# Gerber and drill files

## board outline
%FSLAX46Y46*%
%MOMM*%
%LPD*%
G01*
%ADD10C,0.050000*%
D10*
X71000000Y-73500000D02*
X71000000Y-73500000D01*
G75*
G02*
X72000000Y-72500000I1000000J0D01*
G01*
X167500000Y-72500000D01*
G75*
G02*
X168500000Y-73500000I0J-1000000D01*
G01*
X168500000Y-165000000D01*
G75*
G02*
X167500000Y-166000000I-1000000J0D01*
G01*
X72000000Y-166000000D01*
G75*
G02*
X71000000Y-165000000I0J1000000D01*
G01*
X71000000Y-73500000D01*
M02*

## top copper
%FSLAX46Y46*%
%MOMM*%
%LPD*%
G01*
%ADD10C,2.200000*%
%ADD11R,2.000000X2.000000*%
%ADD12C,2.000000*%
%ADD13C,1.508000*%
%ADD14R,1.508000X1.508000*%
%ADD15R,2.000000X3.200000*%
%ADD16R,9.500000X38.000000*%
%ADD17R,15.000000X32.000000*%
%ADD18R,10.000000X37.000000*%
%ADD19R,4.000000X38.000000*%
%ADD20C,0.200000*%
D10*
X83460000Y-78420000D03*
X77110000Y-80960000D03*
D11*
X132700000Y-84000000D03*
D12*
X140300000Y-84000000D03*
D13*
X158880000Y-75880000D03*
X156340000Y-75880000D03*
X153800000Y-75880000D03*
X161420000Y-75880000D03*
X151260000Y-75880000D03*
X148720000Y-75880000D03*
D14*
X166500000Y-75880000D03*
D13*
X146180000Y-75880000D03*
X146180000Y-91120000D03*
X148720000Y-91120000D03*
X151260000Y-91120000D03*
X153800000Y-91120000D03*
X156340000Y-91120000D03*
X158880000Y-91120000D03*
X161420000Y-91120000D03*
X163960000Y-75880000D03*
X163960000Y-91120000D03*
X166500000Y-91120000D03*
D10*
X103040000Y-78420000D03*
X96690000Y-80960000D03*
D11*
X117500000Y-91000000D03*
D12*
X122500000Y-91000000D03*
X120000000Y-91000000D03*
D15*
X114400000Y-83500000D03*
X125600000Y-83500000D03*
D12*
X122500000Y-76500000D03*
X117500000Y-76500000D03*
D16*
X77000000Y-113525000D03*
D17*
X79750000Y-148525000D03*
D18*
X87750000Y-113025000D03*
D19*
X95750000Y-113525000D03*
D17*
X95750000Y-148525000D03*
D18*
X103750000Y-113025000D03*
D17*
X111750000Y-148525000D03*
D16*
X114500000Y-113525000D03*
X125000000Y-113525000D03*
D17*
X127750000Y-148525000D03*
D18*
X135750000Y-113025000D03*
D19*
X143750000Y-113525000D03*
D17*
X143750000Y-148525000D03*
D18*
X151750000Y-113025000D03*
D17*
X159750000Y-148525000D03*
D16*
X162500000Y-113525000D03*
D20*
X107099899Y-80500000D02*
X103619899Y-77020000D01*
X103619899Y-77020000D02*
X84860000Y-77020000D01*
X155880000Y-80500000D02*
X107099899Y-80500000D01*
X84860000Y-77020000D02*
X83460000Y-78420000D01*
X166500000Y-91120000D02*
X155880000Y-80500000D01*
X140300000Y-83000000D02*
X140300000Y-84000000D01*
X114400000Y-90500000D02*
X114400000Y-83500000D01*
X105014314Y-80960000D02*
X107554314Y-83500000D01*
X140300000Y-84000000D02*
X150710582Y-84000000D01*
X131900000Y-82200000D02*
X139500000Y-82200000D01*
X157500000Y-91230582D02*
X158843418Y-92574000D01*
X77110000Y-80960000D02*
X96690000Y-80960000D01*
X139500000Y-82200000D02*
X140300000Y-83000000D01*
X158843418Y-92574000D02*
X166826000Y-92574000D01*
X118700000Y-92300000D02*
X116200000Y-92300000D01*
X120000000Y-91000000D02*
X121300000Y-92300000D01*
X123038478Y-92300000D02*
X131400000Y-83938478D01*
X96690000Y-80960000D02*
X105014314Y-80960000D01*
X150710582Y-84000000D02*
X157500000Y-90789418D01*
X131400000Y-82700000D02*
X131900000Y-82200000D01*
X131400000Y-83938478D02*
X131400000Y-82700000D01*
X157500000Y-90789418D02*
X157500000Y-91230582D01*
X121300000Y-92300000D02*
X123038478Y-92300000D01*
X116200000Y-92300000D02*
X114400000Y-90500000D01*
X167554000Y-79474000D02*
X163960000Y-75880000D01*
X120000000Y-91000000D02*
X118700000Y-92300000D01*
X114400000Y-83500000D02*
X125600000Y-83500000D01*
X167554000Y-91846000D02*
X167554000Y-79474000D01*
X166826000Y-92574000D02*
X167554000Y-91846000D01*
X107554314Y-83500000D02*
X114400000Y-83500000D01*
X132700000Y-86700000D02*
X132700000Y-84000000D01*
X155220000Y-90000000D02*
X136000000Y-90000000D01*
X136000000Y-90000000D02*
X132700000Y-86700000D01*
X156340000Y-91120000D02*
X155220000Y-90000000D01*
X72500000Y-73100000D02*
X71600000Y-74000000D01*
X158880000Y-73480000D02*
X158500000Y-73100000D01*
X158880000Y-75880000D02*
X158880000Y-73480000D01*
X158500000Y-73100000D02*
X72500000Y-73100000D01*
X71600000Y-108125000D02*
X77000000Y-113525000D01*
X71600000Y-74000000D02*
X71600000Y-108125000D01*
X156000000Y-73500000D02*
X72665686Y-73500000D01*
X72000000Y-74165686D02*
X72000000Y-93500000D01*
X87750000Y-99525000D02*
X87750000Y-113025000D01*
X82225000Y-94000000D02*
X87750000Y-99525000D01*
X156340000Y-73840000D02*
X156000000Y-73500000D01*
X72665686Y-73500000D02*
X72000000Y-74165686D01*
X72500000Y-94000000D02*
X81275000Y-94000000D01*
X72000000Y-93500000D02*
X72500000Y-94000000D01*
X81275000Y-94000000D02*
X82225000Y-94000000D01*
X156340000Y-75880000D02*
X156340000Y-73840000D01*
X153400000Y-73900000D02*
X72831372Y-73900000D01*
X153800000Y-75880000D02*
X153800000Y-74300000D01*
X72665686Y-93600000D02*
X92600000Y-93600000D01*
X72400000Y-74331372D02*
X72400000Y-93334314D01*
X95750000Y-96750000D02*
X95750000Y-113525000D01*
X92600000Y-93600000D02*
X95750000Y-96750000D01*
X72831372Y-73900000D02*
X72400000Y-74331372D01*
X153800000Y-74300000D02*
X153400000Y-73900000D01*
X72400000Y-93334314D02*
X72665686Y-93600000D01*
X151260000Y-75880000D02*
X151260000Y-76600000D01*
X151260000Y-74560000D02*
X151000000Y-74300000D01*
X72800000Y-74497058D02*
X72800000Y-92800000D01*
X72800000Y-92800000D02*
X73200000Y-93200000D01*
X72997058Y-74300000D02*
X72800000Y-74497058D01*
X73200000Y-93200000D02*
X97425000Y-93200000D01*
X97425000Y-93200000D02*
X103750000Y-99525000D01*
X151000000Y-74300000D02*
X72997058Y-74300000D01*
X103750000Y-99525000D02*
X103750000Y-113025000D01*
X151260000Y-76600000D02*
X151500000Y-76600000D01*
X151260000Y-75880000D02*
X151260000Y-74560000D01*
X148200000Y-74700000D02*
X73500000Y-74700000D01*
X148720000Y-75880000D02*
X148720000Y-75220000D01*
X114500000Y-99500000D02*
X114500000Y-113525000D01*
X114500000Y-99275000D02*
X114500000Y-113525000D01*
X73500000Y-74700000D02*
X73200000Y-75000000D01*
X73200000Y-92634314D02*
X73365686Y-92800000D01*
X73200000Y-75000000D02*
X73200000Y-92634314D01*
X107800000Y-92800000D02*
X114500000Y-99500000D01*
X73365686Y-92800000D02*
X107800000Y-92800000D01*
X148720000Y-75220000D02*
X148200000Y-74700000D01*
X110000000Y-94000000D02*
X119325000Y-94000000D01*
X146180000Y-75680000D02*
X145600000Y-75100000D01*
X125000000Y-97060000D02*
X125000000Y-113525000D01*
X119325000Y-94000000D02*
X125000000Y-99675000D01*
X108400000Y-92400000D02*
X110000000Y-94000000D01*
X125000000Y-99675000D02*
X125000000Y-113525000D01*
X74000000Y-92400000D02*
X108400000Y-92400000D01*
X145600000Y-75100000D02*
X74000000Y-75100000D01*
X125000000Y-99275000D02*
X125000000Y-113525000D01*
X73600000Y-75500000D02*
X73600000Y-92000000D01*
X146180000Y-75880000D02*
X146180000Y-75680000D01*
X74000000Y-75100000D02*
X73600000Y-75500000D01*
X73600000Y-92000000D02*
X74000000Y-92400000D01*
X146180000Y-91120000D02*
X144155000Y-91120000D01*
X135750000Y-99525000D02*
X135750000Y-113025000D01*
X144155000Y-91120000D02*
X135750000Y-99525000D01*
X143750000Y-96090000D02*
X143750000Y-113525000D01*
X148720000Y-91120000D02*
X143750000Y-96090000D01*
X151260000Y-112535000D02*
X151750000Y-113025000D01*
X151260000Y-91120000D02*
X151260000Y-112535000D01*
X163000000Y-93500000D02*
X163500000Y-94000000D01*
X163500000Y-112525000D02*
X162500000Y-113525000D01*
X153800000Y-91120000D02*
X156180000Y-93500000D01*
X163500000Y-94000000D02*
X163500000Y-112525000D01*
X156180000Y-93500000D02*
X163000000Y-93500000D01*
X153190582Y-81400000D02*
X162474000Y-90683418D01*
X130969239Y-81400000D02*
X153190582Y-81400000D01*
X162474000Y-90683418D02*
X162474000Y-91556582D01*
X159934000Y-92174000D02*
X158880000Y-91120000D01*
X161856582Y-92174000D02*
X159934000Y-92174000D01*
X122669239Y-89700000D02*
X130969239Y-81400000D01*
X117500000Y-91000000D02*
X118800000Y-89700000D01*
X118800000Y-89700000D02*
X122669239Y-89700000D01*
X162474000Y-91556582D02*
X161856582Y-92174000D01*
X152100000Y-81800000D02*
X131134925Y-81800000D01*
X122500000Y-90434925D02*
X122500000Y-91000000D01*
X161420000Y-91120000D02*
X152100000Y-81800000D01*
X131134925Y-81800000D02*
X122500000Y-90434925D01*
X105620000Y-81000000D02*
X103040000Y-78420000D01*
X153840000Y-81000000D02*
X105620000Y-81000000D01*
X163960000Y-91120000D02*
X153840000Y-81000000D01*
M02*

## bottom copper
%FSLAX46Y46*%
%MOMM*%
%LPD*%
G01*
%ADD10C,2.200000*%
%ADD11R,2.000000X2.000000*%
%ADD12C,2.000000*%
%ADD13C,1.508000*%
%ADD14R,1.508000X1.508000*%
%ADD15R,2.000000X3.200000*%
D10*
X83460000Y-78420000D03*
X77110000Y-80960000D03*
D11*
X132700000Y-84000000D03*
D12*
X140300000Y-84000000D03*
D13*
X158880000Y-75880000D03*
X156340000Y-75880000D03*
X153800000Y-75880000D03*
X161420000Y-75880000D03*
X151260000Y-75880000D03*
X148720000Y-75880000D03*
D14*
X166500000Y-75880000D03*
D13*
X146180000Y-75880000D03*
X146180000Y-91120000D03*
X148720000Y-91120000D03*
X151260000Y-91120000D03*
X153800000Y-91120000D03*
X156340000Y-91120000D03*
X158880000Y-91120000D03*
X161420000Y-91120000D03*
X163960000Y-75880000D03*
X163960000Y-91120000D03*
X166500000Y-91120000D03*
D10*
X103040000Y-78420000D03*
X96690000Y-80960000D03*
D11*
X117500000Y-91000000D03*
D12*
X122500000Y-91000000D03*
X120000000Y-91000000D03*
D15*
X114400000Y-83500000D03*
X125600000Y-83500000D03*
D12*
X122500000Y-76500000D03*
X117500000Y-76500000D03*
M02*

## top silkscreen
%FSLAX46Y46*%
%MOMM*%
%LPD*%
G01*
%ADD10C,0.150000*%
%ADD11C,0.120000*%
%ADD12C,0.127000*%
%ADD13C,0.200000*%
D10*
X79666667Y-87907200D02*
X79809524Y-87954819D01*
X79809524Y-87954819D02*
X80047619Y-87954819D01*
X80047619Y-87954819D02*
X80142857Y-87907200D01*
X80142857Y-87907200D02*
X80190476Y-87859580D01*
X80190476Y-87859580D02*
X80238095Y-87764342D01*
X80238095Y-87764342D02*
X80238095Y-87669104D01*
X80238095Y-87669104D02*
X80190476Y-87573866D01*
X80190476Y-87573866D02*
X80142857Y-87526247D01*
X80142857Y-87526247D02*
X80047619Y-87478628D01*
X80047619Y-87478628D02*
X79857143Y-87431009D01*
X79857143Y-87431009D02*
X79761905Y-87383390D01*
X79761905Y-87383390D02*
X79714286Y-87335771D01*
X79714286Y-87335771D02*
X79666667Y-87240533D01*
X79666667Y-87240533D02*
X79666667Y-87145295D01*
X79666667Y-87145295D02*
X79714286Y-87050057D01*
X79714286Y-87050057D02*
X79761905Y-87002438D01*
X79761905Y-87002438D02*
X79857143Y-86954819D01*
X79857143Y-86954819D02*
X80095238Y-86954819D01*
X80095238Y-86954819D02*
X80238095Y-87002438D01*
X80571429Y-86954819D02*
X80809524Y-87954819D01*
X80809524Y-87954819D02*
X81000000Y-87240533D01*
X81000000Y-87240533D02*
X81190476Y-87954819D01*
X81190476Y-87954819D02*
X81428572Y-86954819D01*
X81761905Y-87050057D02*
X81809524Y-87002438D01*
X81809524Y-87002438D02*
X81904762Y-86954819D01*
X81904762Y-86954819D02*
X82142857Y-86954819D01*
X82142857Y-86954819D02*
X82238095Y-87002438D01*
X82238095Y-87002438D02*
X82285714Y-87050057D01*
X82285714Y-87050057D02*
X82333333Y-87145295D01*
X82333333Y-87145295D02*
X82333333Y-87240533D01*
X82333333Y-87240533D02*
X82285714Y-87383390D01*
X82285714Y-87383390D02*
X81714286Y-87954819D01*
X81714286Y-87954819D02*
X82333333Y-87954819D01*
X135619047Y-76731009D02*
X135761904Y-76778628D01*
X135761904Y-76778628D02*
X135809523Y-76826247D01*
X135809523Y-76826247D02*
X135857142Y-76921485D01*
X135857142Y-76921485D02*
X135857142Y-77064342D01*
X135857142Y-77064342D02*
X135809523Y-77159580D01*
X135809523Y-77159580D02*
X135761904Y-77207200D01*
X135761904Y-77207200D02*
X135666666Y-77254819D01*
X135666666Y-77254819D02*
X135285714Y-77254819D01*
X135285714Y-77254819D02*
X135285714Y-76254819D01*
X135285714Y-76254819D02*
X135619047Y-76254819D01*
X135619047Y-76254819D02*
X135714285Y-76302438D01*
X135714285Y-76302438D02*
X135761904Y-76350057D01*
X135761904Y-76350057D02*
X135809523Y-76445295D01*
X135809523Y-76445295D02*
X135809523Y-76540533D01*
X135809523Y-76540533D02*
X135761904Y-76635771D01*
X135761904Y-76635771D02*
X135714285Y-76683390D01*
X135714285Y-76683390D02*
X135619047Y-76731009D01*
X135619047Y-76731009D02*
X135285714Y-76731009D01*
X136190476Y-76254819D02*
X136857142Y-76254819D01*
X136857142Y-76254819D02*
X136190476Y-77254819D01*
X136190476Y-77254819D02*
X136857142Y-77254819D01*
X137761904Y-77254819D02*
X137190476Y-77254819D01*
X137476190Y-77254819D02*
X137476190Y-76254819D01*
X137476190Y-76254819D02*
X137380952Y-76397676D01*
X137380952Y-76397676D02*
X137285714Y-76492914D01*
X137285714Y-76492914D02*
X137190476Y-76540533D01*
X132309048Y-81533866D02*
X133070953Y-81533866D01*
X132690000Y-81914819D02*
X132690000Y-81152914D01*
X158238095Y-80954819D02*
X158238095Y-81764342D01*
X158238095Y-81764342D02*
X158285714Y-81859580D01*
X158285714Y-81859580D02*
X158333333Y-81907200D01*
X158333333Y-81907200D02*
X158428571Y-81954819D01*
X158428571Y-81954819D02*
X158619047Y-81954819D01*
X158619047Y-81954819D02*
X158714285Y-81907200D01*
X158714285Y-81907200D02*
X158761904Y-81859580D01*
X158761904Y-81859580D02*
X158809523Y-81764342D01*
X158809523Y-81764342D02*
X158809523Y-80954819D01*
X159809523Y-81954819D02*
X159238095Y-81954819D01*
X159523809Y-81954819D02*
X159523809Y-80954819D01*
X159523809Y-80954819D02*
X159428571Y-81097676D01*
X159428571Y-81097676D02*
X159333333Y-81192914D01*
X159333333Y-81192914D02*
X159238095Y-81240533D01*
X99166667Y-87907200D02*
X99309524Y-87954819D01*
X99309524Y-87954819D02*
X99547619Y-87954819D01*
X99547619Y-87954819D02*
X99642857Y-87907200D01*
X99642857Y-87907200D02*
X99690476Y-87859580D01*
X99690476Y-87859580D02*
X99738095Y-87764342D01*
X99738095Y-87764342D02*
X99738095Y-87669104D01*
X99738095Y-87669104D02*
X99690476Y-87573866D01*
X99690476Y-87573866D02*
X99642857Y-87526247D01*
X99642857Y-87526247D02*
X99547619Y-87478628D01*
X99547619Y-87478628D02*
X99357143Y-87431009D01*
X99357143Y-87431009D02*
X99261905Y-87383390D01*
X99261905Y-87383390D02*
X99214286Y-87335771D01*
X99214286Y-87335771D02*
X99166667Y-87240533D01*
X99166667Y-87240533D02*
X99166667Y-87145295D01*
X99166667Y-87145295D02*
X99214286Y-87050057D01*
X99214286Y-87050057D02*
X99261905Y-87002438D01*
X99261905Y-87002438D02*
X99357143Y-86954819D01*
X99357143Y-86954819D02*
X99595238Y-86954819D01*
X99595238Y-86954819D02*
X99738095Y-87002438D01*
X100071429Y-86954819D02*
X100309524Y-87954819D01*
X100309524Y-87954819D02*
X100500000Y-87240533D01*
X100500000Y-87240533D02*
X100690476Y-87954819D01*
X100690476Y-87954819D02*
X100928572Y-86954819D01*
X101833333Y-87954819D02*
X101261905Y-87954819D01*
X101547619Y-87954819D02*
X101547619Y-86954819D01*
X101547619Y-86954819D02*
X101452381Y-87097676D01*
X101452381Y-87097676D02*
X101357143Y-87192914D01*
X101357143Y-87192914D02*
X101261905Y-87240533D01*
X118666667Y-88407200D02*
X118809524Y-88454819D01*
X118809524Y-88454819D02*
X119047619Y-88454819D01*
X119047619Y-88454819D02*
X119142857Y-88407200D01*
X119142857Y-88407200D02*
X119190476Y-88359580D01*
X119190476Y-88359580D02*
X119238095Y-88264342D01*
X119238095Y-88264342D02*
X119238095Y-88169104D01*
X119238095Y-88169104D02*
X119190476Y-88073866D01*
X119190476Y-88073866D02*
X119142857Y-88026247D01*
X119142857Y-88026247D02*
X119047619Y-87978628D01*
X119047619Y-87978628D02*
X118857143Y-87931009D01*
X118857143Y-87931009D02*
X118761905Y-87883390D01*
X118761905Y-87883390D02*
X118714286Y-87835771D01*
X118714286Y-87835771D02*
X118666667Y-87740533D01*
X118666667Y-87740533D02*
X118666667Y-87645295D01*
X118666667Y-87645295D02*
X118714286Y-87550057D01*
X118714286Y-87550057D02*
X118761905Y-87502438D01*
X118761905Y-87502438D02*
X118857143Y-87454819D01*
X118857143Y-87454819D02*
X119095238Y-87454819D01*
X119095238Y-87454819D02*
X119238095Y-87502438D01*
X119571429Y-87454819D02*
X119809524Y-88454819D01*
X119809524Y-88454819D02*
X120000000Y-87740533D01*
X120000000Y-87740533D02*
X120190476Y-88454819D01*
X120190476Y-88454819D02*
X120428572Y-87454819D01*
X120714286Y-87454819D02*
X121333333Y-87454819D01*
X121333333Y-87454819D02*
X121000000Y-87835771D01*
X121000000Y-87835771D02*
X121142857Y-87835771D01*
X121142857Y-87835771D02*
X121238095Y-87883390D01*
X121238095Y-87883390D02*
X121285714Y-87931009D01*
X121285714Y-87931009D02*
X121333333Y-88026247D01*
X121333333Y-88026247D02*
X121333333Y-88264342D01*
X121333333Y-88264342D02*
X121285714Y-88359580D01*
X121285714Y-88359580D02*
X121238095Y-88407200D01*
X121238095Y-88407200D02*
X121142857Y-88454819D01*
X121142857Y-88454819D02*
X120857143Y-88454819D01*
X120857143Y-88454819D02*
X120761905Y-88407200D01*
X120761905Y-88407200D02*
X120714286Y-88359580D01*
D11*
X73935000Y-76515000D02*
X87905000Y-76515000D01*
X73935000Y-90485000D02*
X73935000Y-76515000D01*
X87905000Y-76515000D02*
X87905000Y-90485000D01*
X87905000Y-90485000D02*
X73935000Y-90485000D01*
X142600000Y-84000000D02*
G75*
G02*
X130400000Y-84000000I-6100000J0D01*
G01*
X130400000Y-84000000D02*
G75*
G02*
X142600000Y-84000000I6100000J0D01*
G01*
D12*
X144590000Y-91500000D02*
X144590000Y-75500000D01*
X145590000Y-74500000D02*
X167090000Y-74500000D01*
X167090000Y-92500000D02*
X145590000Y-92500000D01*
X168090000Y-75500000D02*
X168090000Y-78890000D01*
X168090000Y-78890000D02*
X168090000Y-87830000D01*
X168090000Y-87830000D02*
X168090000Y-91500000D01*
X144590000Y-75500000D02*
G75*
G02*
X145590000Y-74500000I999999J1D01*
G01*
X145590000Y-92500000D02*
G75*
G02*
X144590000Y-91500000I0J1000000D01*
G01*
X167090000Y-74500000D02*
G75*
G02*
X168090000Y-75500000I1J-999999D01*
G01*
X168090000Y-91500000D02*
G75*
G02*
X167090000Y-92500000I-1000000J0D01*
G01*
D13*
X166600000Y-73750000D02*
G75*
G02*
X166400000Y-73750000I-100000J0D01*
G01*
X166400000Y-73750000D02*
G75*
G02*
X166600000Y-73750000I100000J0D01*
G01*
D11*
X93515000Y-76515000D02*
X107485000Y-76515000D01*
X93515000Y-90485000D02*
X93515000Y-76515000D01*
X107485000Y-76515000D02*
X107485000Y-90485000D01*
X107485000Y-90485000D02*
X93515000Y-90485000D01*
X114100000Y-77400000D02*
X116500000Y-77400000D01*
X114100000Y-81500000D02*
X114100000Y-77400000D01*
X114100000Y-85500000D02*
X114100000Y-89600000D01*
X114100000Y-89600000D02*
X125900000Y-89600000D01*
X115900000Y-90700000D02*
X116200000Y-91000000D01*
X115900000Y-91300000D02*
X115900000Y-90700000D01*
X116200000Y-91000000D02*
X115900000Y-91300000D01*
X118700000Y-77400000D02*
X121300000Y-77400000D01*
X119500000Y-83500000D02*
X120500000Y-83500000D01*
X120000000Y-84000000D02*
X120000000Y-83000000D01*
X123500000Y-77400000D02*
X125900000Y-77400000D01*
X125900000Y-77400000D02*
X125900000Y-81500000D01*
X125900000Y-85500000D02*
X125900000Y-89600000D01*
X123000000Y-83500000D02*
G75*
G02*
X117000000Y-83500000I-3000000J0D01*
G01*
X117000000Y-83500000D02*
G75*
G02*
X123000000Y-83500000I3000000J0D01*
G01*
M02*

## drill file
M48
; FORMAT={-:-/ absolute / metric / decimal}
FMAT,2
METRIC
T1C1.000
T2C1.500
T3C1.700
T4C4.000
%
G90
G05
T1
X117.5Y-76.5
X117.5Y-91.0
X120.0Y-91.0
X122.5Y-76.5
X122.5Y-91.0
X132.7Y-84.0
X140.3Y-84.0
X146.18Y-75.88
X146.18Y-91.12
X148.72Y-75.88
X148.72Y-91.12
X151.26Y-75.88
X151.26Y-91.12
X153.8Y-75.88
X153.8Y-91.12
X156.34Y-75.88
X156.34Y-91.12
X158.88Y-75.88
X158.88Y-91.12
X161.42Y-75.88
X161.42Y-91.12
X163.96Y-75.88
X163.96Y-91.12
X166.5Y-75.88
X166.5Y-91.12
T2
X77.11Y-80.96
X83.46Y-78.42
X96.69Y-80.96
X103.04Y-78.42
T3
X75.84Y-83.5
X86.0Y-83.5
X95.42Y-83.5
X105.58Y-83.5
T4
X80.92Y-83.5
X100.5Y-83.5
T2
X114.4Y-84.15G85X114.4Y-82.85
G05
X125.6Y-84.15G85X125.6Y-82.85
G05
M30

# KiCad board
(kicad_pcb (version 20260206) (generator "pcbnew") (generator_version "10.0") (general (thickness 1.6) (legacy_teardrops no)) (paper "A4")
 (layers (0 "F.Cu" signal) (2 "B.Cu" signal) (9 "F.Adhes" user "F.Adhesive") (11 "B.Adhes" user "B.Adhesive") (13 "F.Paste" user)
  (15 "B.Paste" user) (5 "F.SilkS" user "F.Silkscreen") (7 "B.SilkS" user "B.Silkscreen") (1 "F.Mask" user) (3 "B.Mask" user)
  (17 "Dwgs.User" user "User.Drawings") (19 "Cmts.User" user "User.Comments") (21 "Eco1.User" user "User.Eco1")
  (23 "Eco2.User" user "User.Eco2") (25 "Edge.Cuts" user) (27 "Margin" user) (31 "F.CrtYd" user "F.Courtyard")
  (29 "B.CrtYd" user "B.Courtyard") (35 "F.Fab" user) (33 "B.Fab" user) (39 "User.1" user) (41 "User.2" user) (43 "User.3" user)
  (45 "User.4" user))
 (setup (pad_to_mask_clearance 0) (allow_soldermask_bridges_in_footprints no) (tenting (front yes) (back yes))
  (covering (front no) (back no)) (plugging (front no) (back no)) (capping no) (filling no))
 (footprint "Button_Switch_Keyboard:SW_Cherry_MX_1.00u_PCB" (layer "F.Cu") (at 83.46 78.42)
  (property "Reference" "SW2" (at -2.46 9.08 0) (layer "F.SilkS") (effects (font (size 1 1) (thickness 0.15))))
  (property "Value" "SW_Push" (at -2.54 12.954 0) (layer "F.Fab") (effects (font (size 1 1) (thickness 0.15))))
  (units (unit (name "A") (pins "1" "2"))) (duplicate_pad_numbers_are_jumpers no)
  (fp_line (start -9.525 -1.905) (end 4.445 -1.905) (stroke (width 0.12) (type solid)) (layer "F.SilkS"))
  (fp_line (start -9.525 12.065) (end -9.525 -1.905) (stroke (width 0.12) (type solid)) (layer "F.SilkS"))
  (fp_line (start 4.445 -1.905) (end 4.445 12.065) (stroke (width 0.12) (type solid)) (layer "F.SilkS"))
  (fp_line (start 4.445 12.065) (end -9.525 12.065) (stroke (width 0.12) (type solid)) (layer "F.SilkS"))
  (pad "" np_thru_hole circle (at -7.62 5.08) (size 1.7 1.7) (drill 1.7) (layers "*.Cu" "*.Mask"))
  (pad "" np_thru_hole circle (at -2.54 5.08) (size 4 4) (drill 4) (layers "*.Cu" "*.Mask"))
  (pad "" np_thru_hole circle (at 2.54 5.08) (size 1.7 1.7) (drill 1.7) (layers "*.Cu" "*.Mask"))
  (pad "1" thru_hole circle (at 0 0) (size 2.2 2.2) (drill 1.5) (layers "*.Cu" "*.Mask") (remove_unused_layers no) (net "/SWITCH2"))
  (pad "2" thru_hole circle (at -6.35 2.54) (size 2.2 2.2) (drill 1.5) (layers "*.Cu" "*.Mask") (remove_unused_layers no) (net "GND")))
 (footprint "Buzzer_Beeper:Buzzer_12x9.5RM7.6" (layer "F.Cu") (at 132.7 84)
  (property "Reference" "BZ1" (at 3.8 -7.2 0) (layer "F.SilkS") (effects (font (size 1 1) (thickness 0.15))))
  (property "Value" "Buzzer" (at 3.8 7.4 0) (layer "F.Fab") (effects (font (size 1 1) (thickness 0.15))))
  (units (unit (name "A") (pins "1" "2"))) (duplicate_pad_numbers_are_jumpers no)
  (fp_circle (center 3.8 0) (end 9.9 0) (stroke (width 0.12) (type solid)) (fill no) (layer "F.SilkS"))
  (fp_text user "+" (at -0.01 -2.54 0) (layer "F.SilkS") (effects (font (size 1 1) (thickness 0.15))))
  (pad "1" thru_hole rect (at 0 0) (size 2 2) (drill 1) (layers "*.Cu" "*.Mask") (remove_unused_layers no) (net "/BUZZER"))
  (pad "2" thru_hole circle (at 7.6 0) (size 2 2) (drill 1) (layers "*.Cu" "*.Mask") (remove_unused_layers no) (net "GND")))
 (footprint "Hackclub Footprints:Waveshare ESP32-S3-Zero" (layer "F.Cu") (at 156.34 83.5 -90)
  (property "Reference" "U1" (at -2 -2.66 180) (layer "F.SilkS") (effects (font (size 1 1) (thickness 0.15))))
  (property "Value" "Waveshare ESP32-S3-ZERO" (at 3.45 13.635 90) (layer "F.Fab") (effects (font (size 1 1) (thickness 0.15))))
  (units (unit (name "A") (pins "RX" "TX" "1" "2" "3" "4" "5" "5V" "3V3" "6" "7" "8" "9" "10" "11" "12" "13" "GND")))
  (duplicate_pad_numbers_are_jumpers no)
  (fp_line (start 8 11.75) (end -8 11.75) (stroke (width 0.127) (type solid)) (layer "F.SilkS"))
  (fp_line (start -9 10.75) (end -9 -10.75) (stroke (width 0.127) (type solid)) (layer "F.SilkS"))
  (fp_line (start 9 -10.75) (end 9 10.75) (stroke (width 0.127) (type solid)) (layer "F.SilkS"))
  (fp_line (start -8 -11.75) (end -4.61 -11.75) (stroke (width 0.127) (type solid)) (layer "F.SilkS"))
  (fp_line (start -4.61 -11.75) (end 4.33 -11.75) (stroke (width 0.127) (type solid)) (layer "F.SilkS"))
  (fp_line (start 4.33 -11.75) (end 8 -11.75) (stroke (width 0.127) (type solid)) (layer "F.SilkS"))
  (fp_arc (start -8 11.75) (mid -8.707107 11.457107) (end -9 10.75) (stroke (width 0.127) (type solid)) (layer "F.SilkS"))
  (fp_arc (start 9 10.75) (mid 8.707107 11.457107) (end 8 11.75) (stroke (width 0.127) (type solid)) (layer "F.SilkS"))
  (fp_arc (start -9 -10.75) (mid -8.707107 -11.457107) (end -8 -11.75) (stroke (width 0.127) (type solid)) (layer "F.SilkS"))
  (fp_arc (start 8 -11.75) (mid 8.707107 -11.457107) (end 9 -10.75) (stroke (width 0.127) (type solid)) (layer "F.SilkS"))
  (fp_circle (center -9.75 -10.16) (end -9.65 -10.16) (stroke (width 0.2) (type solid)) (fill no) (layer "F.SilkS"))
  (pad "1" thru_hole circle (at -7.62 -2.54 270) (size 1.508 1.508) (drill 1) (layers "*.Cu" "*.Mask") (remove_unused_layers no)
   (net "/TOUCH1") (solder_mask_margin 0.102))
  (pad "2" thru_hole circle (at -7.62 0 270) (size 1.508 1.508) (drill 1) (layers "*.Cu" "*.Mask") (remove_unused_layers no) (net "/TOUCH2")
   (solder_mask_margin 0.102))
  (pad "3" thru_hole circle (at -7.62 2.54 270) (size 1.508 1.508) (drill 1) (layers "*.Cu" "*.Mask") (remove_unused_layers no)
   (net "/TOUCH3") (solder_mask_margin 0.102))
  (pad "3V3" thru_hole circle (at -7.62 -5.08 270) (size 1.508 1.508) (drill 1) (layers "*.Cu" "*.Mask") (remove_unused_layers no)
   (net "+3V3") (solder_mask_margin 0.102))
  (pad "4" thru_hole circle (at -7.62 5.08 270) (size 1.508 1.508) (drill 1) (layers "*.Cu" "*.Mask") (remove_unused_layers no)
   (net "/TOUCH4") (solder_mask_margin 0.102))
  (pad "5" thru_hole circle (at -7.62 7.62 270) (size 1.508 1.508) (drill 1) (layers "*.Cu" "*.Mask") (remove_unused_layers no)
   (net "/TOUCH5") (solder_mask_margin 0.102))
  (pad "5V" thru_hole rect (at -7.62 -10.16 270) (size 1.508 1.508) (drill 1) (layers "*.Cu" "*.Mask") (remove_unused_layers no) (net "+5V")
   (solder_mask_margin 0.102))
  (pad "6" thru_hole circle (at -7.62 10.16 270) (size 1.508 1.508) (drill 1) (layers "*.Cu" "*.Mask") (remove_unused_layers no)
   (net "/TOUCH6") (solder_mask_margin 0.102))
  (pad "7" thru_hole circle (at 7.62 10.16 270) (size 1.508 1.508) (drill 1) (layers "*.Cu" "*.Mask") (remove_unused_layers no)
   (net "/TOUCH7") (solder_mask_margin 0.102))
  (pad "8" thru_hole circle (at 7.62 7.62 270) (size 1.508 1.508) (drill 1) (layers "*.Cu" "*.Mask") (remove_unused_layers no)
   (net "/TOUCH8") (solder_mask_margin 0.102))
  (pad "9" thru_hole circle (at 7.62 5.08 270) (size 1.508 1.508) (drill 1) (layers "*.Cu" "*.Mask") (remove_unused_layers no)
   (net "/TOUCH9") (solder_mask_margin 0.102))
  (pad "10" thru_hole circle (at 7.62 2.54 270) (size 1.508 1.508) (drill 1) (layers "*.Cu" "*.Mask") (remove_unused_layers no)
   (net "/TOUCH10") (solder_mask_margin 0.102))
  (pad "11" thru_hole circle (at 7.62 0 270) (size 1.508 1.508) (drill 1) (layers "*.Cu" "*.Mask") (remove_unused_layers no) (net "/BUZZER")
   (solder_mask_margin 0.102))
  (pad "12" thru_hole circle (at 7.62 -2.54 270) (size 1.508 1.508) (drill 1) (layers "*.Cu" "*.Mask") (remove_unused_layers no)
   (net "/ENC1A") (solder_mask_margin 0.102))
  (pad "13" thru_hole circle (at 7.62 -5.08 270) (size 1.508 1.508) (drill 1) (layers "*.Cu" "*.Mask") (remove_unused_layers no)
   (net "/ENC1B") (solder_mask_margin 0.102))
  (pad "GND" thru_hole circle (at -7.62 -7.62 270) (size 1.508 1.508) (drill 1) (layers "*.Cu" "*.Mask") (remove_unused_layers no)
   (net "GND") (solder_mask_margin 0.102))
  (pad "RX" thru_hole circle (at 7.62 -7.62 270) (size 1.508 1.508) (drill 1) (layers "*.Cu" "*.Mask") (remove_unused_layers no)
   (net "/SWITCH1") (solder_mask_margin 0.102))
  (pad "TX" thru_hole circle (at 7.62 -10.16 270) (size 1.508 1.508) (drill 1) (layers "*.Cu" "*.Mask") (remove_unused_layers no)
   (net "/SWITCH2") (solder_mask_margin 0.102)))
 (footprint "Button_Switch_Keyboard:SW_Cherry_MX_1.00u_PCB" (layer "F.Cu") (at 103.04 78.42)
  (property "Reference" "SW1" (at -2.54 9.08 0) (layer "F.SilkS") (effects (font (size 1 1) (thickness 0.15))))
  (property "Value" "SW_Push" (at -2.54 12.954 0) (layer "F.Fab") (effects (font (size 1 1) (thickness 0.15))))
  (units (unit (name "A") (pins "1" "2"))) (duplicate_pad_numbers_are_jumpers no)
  (fp_line (start -9.525 -1.905) (end 4.445 -1.905) (stroke (width 0.12) (type solid)) (layer "F.SilkS"))
  (fp_line (start -9.525 12.065) (end -9.525 -1.905) (stroke (width 0.12) (type solid)) (layer "F.SilkS"))
  (fp_line (start 4.445 -1.905) (end 4.445 12.065) (stroke (width 0.12) (type solid)) (layer "F.SilkS"))
  (fp_line (start 4.445 12.065) (end -9.525 12.065) (stroke (width 0.12) (type solid)) (layer "F.SilkS"))
  (pad "" np_thru_hole circle (at -7.62 5.08) (size 1.7 1.7) (drill 1.7) (layers "*.Cu" "*.Mask"))
  (pad "" np_thru_hole circle (at -2.54 5.08) (size 4 4) (drill 4) (layers "*.Cu" "*.Mask"))
  (pad "" np_thru_hole circle (at 2.54 5.08) (size 1.7 1.7) (drill 1.7) (layers "*.Cu" "*.Mask"))
  (pad "1" thru_hole circle (at 0 0) (size 2.2 2.2) (drill 1.5) (layers "*.Cu" "*.Mask") (remove_unused_layers no) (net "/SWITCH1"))
  (pad "2" thru_hole circle (at -6.35 2.54) (size 2.2 2.2) (drill 1.5) (layers "*.Cu" "*.Mask") (remove_unused_layers no) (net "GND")))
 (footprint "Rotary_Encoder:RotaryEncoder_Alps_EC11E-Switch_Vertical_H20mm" (layer "F.Cu") (at 117.5 91 90)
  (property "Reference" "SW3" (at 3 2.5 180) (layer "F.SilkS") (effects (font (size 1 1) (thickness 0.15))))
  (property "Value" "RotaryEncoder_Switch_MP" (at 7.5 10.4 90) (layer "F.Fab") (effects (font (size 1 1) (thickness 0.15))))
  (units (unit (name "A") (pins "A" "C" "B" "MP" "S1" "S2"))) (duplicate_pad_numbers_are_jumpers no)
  (fp_line (start 13.6 -3.4) (end 13.6 -1) (stroke (width 0.12) (type solid)) (layer "F.SilkS"))
  (fp_line (start 9.5 -3.4) (end 13.6 -3.4) (stroke (width 0.12) (type solid)) (layer "F.SilkS"))
  (fp_line (start 5.5 -3.4) (end 1.4 -3.4) (stroke (width 0.12) (type solid)) (layer "F.SilkS"))
  (fp_line (start 1.4 -3.4) (end 1.4 8.4) (stroke (width 0.12) (type solid)) (layer "F.SilkS"))
  (fp_line (start 0.3 -1.6) (end 0 -1.3) (stroke (width 0.12) (type solid)) (layer "F.SilkS"))
  (fp_line (start -0.3 -1.6) (end 0.3 -1.6) (stroke (width 0.12) (type solid)) (layer "F.SilkS"))
  (fp_line (start 0 -1.3) (end -0.3 -1.6) (stroke (width 0.12) (type solid)) (layer "F.SilkS"))
  (fp_line (start 13.6 1.2) (end 13.6 3.8) (stroke (width 0.12) (type solid)) (layer "F.SilkS"))
  (fp_line (start 7.5 2) (end 7.5 3) (stroke (width 0.12) (type solid)) (layer "F.SilkS"))
  (fp_line (start 7 2.5) (end 8 2.5) (stroke (width 0.12) (type solid)) (layer "F.SilkS"))
  (fp_line (start 13.6 6) (end 13.6 8.4) (stroke (width 0.12) (type solid)) (layer "F.SilkS"))
  (fp_line (start 13.6 8.4) (end 9.5 8.4) (stroke (width 0.12) (type solid)) (layer "F.SilkS"))
  (fp_line (start 5.5 8.4) (end 1.4 8.4) (stroke (width 0.12) (type solid)) (layer "F.SilkS"))
  (fp_circle (center 7.5 2.5) (end 10.5 2.5) (stroke (width 0.12) (type solid)) (fill no) (layer "F.SilkS"))
  (pad "A" thru_hole rect (at 0 0 90) (size 2 2) (drill 1) (layers "*.Cu" "*.Mask") (remove_unused_layers no) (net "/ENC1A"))
  (pad "B" thru_hole circle (at 0 5 90) (size 2 2) (drill 1) (layers "*.Cu" "*.Mask") (remove_unused_layers no) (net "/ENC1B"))
  (pad "C" thru_hole circle (at 0 2.5 90) (size 2 2) (drill 1) (layers "*.Cu" "*.Mask") (remove_unused_layers no) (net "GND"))
  (pad "MP" thru_hole rect (at 7.5 -3.1 90) (size 3.2 2) (drill oval 2.8 1.5) (layers "*.Cu" "*.Mask") (remove_unused_layers no) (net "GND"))
  (pad "MP" thru_hole rect (at 7.5 8.1 90) (size 3.2 2) (drill oval 2.8 1.5) (layers "*.Cu" "*.Mask") (remove_unused_layers no) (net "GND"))
  (pad "S1" thru_hole circle (at 14.5 5 90) (size 2 2) (drill 1) (layers "*.Cu" "*.Mask") (remove_unused_layers no)
   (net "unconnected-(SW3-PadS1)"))
  (pad "S2" thru_hole circle (at 14.5 0 90) (size 2 2) (drill 1) (layers "*.Cu" "*.Mask") (remove_unused_layers no)
   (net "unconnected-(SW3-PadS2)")))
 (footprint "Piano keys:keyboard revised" (layer "F.Cu") (at 67.75 111.525)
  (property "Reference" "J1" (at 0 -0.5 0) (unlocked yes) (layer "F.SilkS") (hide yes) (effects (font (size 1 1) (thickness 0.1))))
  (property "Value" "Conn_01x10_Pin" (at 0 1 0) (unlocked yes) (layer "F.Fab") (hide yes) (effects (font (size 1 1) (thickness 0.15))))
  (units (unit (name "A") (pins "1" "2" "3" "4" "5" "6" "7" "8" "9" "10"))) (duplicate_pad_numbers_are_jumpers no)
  (pad "1" smd rect (at 9.25 2) (size 9.5 38) (layers "F.Cu" "F.Mask") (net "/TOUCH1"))
  (pad "1" smd rect (at 12 37) (size 15 32) (layers "F.Cu" "F.Mask") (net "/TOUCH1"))
  (pad "2" smd rect (at 20 1.5) (size 10 37) (layers "F.Cu" "F.Mask") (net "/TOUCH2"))
  (pad "3" smd rect (at 28 2) (size 4 38) (layers "F.Cu" "F.Mask") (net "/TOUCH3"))
  (pad "3" smd rect (at 28 37) (size 15 32) (layers "F.Cu" "F.Mask") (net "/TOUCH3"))
  (pad "4" smd rect (at 36 1.5) (size 10 37) (layers "F.Cu" "F.Mask") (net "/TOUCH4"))
  (pad "5" smd rect (at 44 37) (size 15 32) (layers "F.Cu" "F.Mask") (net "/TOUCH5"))
  (pad "5" smd rect (at 46.75 2) (size 9.5 38) (layers "F.Cu" "F.Mask") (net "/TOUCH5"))
  (pad "6" smd rect (at 57.25 2) (size 9.5 38) (layers "F.Cu" "F.Mask") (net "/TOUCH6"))
  (pad "6" smd rect (at 60 37) (size 15 32) (layers "F.Cu" "F.Mask") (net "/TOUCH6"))
  (pad "7" smd rect (at 68 1.5) (size 10 37) (layers "F.Cu" "F.Mask") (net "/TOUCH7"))
  (pad "8" smd rect (at 76 2) (size 4 38) (layers "F.Cu" "F.Mask") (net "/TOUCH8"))
  (pad "8" smd rect (at 76 37) (size 15 32) (layers "F.Cu" "F.Mask") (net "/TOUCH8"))
  (pad "9" smd rect (at 84 1.5) (size 10 37) (layers "F.Cu" "F.Mask") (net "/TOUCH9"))
  (pad "10" smd rect (at 92 37) (size 15 32) (layers "F.Cu" "F.Mask") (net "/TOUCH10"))
  (pad "10" smd rect (at 94.75 2) (size 9.5 38) (layers "F.Cu" "F.Mask") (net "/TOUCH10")))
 (gr_rect (start 71 72.5) (end 168.5 166) (radius 1) (stroke (width 0.05) (type solid)) (fill no) (layer "Edge.Cuts"))
 (segment (start 107.099899 80.5) (end 103.619899 77.02) (width 0.2) (layer "F.Cu") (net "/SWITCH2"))
 (segment (start 103.619899 77.02) (end 84.86 77.02) (width 0.2) (layer "F.Cu") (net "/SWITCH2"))
 (segment (start 155.88 80.5) (end 107.099899 80.5) (width 0.2) (layer "F.Cu") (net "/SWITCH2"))
 (segment (start 84.86 77.02) (end 83.46 78.42) (width 0.2) (layer "F.Cu") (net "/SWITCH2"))
 (segment (start 166.5 91.12) (end 155.88 80.5) (width 0.2) (layer "F.Cu") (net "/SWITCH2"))
 (segment (start 140.3 83) (end 140.3 84) (width 0.2) (layer "F.Cu") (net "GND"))
 (segment (start 114.4 90.5) (end 114.4 83.5) (width 0.2) (layer "F.Cu") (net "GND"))
 (segment (start 105.014314 80.96) (end 107.554314 83.5) (width 0.2) (layer "F.Cu") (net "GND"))
 (segment (start 140.3 84) (end 150.710582 84) (width 0.2) (layer "F.Cu") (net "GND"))
 (segment (start 131.9 82.2) (end 139.5 82.2) (width 0.2) (layer "F.Cu") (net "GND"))
 (segment (start 157.5 91.230582) (end 158.843418 92.574) (width 0.2) (layer "F.Cu") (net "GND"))
 (segment (start 77.11 80.96) (end 96.69 80.96) (width 0.2) (layer "F.Cu") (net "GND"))
 (segment (start 139.5 82.2) (end 140.3 83) (width 0.2) (layer "F.Cu") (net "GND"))
 (segment (start 158.843418 92.574) (end 166.826 92.574) (width 0.2) (layer "F.Cu") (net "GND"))
 (segment (start 118.7 92.3) (end 116.2 92.3) (width 0.2) (layer "F.Cu") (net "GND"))
 (segment (start 120 91) (end 121.3 92.3) (width 0.2) (layer "F.Cu") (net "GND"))
 (segment (start 123.038478 92.3) (end 131.4 83.938478) (width 0.2) (layer "F.Cu") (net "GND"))
 (segment (start 96.69 80.96) (end 105.014314 80.96) (width 0.2) (layer "F.Cu") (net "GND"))
 (segment (start 150.710582 84) (end 157.5 90.789418) (width 0.2) (layer "F.Cu") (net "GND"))
 (segment (start 131.4 82.7) (end 131.9 82.2) (width 0.2) (layer "F.Cu") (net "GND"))
 (segment (start 131.4 83.938478) (end 131.4 82.7) (width 0.2) (layer "F.Cu") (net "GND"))
 (segment (start 157.5 90.789418) (end 157.5 91.230582) (width 0.2) (layer "F.Cu") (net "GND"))
 (segment (start 121.3 92.3) (end 123.038478 92.3) (width 0.2) (layer "F.Cu") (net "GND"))
 (segment (start 116.2 92.3) (end 114.4 90.5) (width 0.2) (layer "F.Cu") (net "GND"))
 (segment (start 167.554 79.474) (end 163.96 75.88) (width 0.2) (layer "F.Cu") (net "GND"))
 (segment (start 120 91) (end 118.7 92.3) (width 0.2) (layer "F.Cu") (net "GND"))
 (segment (start 114.4 83.5) (end 125.6 83.5) (width 0.2) (layer "F.Cu") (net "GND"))
 (segment (start 167.554 91.846) (end 167.554 79.474) (width 0.2) (layer "F.Cu") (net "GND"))
 (segment (start 166.826 92.574) (end 167.554 91.846) (width 0.2) (layer "F.Cu") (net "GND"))
 (segment (start 107.554314 83.5) (end 114.4 83.5) (width 0.2) (layer "F.Cu") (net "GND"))
 (segment (start 132.7 86.7) (end 132.7 84) (width 0.2) (layer "F.Cu") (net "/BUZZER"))
 (segment (start 155.22 90) (end 136 90) (width 0.2) (layer "F.Cu") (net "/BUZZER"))
 (segment (start 136 90) (end 132.7 86.7) (width 0.2) (layer "F.Cu") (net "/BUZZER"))
 (segment (start 156.34 91.12) (end 155.22 90) (width 0.2) (layer "F.Cu") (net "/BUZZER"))
 (segment (start 72.5 73.1) (end 71.6 74) (width 0.2) (layer "F.Cu") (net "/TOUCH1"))
 (segment (start 158.88 73.48) (end 158.5 73.1) (width 0.2) (layer "F.Cu") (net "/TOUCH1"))
 (segment (start 158.88 75.88) (end 158.88 73.48) (width 0.2) (layer "F.Cu") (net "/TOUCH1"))
 (segment (start 158.5 73.1) (end 72.5 73.1) (width 0.2) (layer "F.Cu") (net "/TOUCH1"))
 (segment (start 71.6 108.125) (end 77 113.525) (width 0.2) (layer "F.Cu") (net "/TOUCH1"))
 (segment (start 71.6 74) (end 71.6 108.125) (width 0.2) (layer "F.Cu") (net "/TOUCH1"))
 (segment (start 156 73.5) (end 72.665686 73.5) (width 0.2) (layer "F.Cu") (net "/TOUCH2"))
 (segment (start 72 74.165686) (end 72 93.5) (width 0.2) (layer "F.Cu") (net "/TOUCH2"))
 (segment (start 87.75 99.525) (end 87.75 113.025) (width 0.2) (layer "F.Cu") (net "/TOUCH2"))
 (segment (start 82.225 94) (end 87.75 99.525) (width 0.2) (layer "F.Cu") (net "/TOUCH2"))
 (segment (start 156.34 73.84) (end 156 73.5) (width 0.2) (layer "F.Cu") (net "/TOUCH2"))
 (segment (start 72.665686 73.5) (end 72 74.165686) (width 0.2) (layer "F.Cu") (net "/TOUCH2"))
 (segment (start 72.5 94) (end 81.275 94) (width 0.2) (layer "F.Cu") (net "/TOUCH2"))
 (segment (start 72 93.5) (end 72.5 94) (width 0.2) (layer "F.Cu") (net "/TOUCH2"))
 (segment (start 81.275 94) (end 82.225 94) (width 0.2) (layer "F.Cu") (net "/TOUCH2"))
 (segment (start 156.34 75.88) (end 156.34 73.84) (width 0.2) (layer "F.Cu") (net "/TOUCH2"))
 (segment (start 153.4 73.9) (end 72.831372 73.9) (width 0.2) (layer "F.Cu") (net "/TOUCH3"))
 (segment (start 153.8 75.88) (end 153.8 74.3) (width 0.2) (layer "F.Cu") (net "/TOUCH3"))
 (segment (start 72.665686 93.6) (end 92.6 93.6) (width 0.2) (layer "F.Cu") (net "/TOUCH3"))
 (segment (start 72.4 74.331372) (end 72.4 93.334314) (width 0.2) (layer "F.Cu") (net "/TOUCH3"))
 (segment (start 95.75 96.75) (end 95.75 113.525) (width 0.2) (layer "F.Cu") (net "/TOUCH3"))
 (segment (start 92.6 93.6) (end 95.75 96.75) (width 0.2) (layer "F.Cu") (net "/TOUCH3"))
 (segment (start 72.831372 73.9) (end 72.4 74.331372) (width 0.2) (layer "F.Cu") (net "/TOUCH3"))
 (segment (start 153.8 74.3) (end 153.4 73.9) (width 0.2) (layer "F.Cu") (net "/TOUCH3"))
 (segment (start 72.4 93.334314) (end 72.665686 93.6) (width 0.2) (layer "F.Cu") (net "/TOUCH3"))
 (segment (start 151.26 75.88) (end 151.26 76.6) (width 0.2) (layer "F.Cu") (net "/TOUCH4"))
 (segment (start 151.26 74.56) (end 151 74.3) (width 0.2) (layer "F.Cu") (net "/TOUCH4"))
 (segment (start 72.8 74.497058) (end 72.8 92.8) (width 0.2) (layer "F.Cu") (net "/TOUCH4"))
 (segment (start 72.8 92.8) (end 73.2 93.2) (width 0.2) (layer "F.Cu") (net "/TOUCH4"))
 (segment (start 72.997058 74.3) (end 72.8 74.497058) (width 0.2) (layer "F.Cu") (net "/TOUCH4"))
 (segment (start 73.2 93.2) (end 97.425 93.2) (width 0.2) (layer "F.Cu") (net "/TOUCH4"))
 (segment (start 97.425 93.2) (end 103.75 99.525) (width 0.2) (layer "F.Cu") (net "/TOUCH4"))
 (segment (start 151 74.3) (end 72.997058 74.3) (width 0.2) (layer "F.Cu") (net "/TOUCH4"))
 (segment (start 103.75 99.525) (end 103.75 113.025) (width 0.2) (layer "F.Cu") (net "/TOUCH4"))
 (segment (start 151.26 76.6) (end 151.5 76.6) (width 0.2) (layer "F.Cu") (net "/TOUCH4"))
 (segment (start 151.26 75.88) (end 151.26 74.56) (width 0.2) (layer "F.Cu") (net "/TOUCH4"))
 (segment (start 148.2 74.7) (end 73.5 74.7) (width 0.2) (layer "F.Cu") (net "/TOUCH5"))
 (segment (start 148.72 75.88) (end 148.72 75.22) (width 0.2) (layer "F.Cu") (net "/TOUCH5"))
 (segment (start 114.5 99.5) (end 114.5 113.525) (width 0.2) (layer "F.Cu") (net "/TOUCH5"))
 (segment (start 114.5 99.275) (end 114.5 113.525) (width 0.2) (layer "F.Cu") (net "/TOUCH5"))
 (segment (start 73.5 74.7) (end 73.2 75) (width 0.2) (layer "F.Cu") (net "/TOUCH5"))
 (segment (start 73.2 92.634314) (end 73.365686 92.8) (width 0.2) (layer "F.Cu") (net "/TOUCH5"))
 (segment (start 73.2 75) (end 73.2 92.634314) (width 0.2) (layer "F.Cu") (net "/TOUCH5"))
 (segment (start 107.8 92.8) (end 114.5 99.5) (width 0.2) (layer "F.Cu") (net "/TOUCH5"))
 (segment (start 73.365686 92.8) (end 107.8 92.8) (width 0.2) (layer "F.Cu") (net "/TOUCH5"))
 (segment (start 148.72 75.22) (end 148.2 74.7) (width 0.2) (layer "F.Cu") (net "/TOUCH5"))
 (segment (start 110 94) (end 119.325 94) (width 0.2) (layer "F.Cu") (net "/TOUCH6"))
 (segment (start 146.18 75.68) (end 145.6 75.1) (width 0.2) (layer "F.Cu") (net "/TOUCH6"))
 (segment (start 125 97.06) (end 125 113.525) (width 0.2) (layer "F.Cu") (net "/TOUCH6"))
 (segment (start 119.325 94) (end 125 99.675) (width 0.2) (layer "F.Cu") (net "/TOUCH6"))
 (segment (start 108.4 92.4) (end 110 94) (width 0.2) (layer "F.Cu") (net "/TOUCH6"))
 (segment (start 125 99.675) (end 125 113.525) (width 0.2) (layer "F.Cu") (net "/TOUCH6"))
 (segment (start 74 92.4) (end 108.4 92.4) (width 0.2) (layer "F.Cu") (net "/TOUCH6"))
 (segment (start 145.6 75.1) (end 74 75.1) (width 0.2) (layer "F.Cu") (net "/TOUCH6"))
 (segment (start 125 99.275) (end 125 113.525) (width 0.2) (layer "F.Cu") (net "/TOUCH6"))
 (segment (start 73.6 75.5) (end 73.6 92) (width 0.2) (layer "F.Cu") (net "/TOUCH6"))
 (segment (start 146.18 75.88) (end 146.18 75.68) (width 0.2) (layer "F.Cu") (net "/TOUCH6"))
 (segment (start 74 75.1) (end 73.6 75.5) (width 0.2) (layer "F.Cu") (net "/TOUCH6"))
 (segment (start 73.6 92) (end 74 92.4) (width 0.2) (layer "F.Cu") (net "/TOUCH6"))
 (segment (start 146.18 91.12) (end 144.155 91.12) (width 0.2) (layer "F.Cu") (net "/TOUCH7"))
 (segment (start 135.75 99.525) (end 135.75 113.025) (width 0.2) (layer "F.Cu") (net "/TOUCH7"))
 (segment (start 144.155 91.12) (end 135.75 99.525) (width 0.2) (layer "F.Cu") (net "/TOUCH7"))
 (segment (start 143.75 96.09) (end 143.75 113.525) (width 0.2) (layer "F.Cu") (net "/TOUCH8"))
 (segment (start 148.72 91.12) (end 143.75 96.09) (width 0.2) (layer "F.Cu") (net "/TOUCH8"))
 (segment (start 151.26 112.535) (end 151.75 113.025) (width 0.2) (layer "F.Cu") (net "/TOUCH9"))
 (segment (start 151.26 91.12) (end 151.26 112.535) (width 0.2) (layer "F.Cu") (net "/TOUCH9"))
 (segment (start 163 93.5) (end 163.5 94) (width 0.2) (layer "F.Cu") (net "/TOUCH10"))
 (segment (start 163.5 112.525) (end 162.5 113.525) (width 0.2) (layer "F.Cu") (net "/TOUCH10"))
 (segment (start 153.8 91.12) (end 156.18 93.5) (width 0.2) (layer "F.Cu") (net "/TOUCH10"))
 (segment (start 163.5 94) (end 163.5 112.525) (width 0.2) (layer "F.Cu") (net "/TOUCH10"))
 (segment (start 156.18 93.5) (end 163 93.5) (width 0.2) (layer "F.Cu") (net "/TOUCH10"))
 (segment (start 153.190582 81.4) (end 162.474 90.683418) (width 0.2) (layer "F.Cu") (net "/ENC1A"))
 (segment (start 130.969239 81.4) (end 153.190582 81.4) (width 0.2) (layer "F.Cu") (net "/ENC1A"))
 (segment (start 162.474 90.683418) (end 162.474 91.556582) (width 0.2) (layer "F.Cu") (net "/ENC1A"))
 (segment (start 159.934 92.174) (end 158.88 91.12) (width 0.2) (layer "F.Cu") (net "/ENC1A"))
 (segment (start 161.856582 92.174) (end 159.934 92.174) (width 0.2) (layer "F.Cu") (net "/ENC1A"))
 (segment (start 122.669239 89.7) (end 130.969239 81.4) (width 0.2) (layer "F.Cu") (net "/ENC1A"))
 (segment (start 117.5 91) (end 118.8 89.7) (width 0.2) (layer "F.Cu") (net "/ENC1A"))
 (segment (start 118.8 89.7) (end 122.669239 89.7) (width 0.2) (layer "F.Cu") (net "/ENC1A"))
 (segment (start 162.474 91.556582) (end 161.856582 92.174) (width 0.2) (layer "F.Cu") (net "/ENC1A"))
 (segment (start 152.1 81.8) (end 131.134925 81.8) (width 0.2) (layer "F.Cu") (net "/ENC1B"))
 (segment (start 122.5 90.434925) (end 122.5 91) (width 0.2) (layer "F.Cu") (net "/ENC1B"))
 (segment (start 161.42 91.12) (end 152.1 81.8) (width 0.2) (layer "F.Cu") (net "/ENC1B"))
 (segment (start 131.134925 81.8) (end 122.5 90.434925) (width 0.2) (layer "F.Cu") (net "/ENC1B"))
 (segment (start 105.62 81) (end 103.04 78.42) (width 0.2) (layer "F.Cu") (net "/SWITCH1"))
 (segment (start 153.84 81) (end 105.62 81) (width 0.2) (layer "F.Cu") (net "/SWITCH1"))
 (segment (start 163.96 91.12) (end 153.84 81) (width 0.2) (layer "F.Cu") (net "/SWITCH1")))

